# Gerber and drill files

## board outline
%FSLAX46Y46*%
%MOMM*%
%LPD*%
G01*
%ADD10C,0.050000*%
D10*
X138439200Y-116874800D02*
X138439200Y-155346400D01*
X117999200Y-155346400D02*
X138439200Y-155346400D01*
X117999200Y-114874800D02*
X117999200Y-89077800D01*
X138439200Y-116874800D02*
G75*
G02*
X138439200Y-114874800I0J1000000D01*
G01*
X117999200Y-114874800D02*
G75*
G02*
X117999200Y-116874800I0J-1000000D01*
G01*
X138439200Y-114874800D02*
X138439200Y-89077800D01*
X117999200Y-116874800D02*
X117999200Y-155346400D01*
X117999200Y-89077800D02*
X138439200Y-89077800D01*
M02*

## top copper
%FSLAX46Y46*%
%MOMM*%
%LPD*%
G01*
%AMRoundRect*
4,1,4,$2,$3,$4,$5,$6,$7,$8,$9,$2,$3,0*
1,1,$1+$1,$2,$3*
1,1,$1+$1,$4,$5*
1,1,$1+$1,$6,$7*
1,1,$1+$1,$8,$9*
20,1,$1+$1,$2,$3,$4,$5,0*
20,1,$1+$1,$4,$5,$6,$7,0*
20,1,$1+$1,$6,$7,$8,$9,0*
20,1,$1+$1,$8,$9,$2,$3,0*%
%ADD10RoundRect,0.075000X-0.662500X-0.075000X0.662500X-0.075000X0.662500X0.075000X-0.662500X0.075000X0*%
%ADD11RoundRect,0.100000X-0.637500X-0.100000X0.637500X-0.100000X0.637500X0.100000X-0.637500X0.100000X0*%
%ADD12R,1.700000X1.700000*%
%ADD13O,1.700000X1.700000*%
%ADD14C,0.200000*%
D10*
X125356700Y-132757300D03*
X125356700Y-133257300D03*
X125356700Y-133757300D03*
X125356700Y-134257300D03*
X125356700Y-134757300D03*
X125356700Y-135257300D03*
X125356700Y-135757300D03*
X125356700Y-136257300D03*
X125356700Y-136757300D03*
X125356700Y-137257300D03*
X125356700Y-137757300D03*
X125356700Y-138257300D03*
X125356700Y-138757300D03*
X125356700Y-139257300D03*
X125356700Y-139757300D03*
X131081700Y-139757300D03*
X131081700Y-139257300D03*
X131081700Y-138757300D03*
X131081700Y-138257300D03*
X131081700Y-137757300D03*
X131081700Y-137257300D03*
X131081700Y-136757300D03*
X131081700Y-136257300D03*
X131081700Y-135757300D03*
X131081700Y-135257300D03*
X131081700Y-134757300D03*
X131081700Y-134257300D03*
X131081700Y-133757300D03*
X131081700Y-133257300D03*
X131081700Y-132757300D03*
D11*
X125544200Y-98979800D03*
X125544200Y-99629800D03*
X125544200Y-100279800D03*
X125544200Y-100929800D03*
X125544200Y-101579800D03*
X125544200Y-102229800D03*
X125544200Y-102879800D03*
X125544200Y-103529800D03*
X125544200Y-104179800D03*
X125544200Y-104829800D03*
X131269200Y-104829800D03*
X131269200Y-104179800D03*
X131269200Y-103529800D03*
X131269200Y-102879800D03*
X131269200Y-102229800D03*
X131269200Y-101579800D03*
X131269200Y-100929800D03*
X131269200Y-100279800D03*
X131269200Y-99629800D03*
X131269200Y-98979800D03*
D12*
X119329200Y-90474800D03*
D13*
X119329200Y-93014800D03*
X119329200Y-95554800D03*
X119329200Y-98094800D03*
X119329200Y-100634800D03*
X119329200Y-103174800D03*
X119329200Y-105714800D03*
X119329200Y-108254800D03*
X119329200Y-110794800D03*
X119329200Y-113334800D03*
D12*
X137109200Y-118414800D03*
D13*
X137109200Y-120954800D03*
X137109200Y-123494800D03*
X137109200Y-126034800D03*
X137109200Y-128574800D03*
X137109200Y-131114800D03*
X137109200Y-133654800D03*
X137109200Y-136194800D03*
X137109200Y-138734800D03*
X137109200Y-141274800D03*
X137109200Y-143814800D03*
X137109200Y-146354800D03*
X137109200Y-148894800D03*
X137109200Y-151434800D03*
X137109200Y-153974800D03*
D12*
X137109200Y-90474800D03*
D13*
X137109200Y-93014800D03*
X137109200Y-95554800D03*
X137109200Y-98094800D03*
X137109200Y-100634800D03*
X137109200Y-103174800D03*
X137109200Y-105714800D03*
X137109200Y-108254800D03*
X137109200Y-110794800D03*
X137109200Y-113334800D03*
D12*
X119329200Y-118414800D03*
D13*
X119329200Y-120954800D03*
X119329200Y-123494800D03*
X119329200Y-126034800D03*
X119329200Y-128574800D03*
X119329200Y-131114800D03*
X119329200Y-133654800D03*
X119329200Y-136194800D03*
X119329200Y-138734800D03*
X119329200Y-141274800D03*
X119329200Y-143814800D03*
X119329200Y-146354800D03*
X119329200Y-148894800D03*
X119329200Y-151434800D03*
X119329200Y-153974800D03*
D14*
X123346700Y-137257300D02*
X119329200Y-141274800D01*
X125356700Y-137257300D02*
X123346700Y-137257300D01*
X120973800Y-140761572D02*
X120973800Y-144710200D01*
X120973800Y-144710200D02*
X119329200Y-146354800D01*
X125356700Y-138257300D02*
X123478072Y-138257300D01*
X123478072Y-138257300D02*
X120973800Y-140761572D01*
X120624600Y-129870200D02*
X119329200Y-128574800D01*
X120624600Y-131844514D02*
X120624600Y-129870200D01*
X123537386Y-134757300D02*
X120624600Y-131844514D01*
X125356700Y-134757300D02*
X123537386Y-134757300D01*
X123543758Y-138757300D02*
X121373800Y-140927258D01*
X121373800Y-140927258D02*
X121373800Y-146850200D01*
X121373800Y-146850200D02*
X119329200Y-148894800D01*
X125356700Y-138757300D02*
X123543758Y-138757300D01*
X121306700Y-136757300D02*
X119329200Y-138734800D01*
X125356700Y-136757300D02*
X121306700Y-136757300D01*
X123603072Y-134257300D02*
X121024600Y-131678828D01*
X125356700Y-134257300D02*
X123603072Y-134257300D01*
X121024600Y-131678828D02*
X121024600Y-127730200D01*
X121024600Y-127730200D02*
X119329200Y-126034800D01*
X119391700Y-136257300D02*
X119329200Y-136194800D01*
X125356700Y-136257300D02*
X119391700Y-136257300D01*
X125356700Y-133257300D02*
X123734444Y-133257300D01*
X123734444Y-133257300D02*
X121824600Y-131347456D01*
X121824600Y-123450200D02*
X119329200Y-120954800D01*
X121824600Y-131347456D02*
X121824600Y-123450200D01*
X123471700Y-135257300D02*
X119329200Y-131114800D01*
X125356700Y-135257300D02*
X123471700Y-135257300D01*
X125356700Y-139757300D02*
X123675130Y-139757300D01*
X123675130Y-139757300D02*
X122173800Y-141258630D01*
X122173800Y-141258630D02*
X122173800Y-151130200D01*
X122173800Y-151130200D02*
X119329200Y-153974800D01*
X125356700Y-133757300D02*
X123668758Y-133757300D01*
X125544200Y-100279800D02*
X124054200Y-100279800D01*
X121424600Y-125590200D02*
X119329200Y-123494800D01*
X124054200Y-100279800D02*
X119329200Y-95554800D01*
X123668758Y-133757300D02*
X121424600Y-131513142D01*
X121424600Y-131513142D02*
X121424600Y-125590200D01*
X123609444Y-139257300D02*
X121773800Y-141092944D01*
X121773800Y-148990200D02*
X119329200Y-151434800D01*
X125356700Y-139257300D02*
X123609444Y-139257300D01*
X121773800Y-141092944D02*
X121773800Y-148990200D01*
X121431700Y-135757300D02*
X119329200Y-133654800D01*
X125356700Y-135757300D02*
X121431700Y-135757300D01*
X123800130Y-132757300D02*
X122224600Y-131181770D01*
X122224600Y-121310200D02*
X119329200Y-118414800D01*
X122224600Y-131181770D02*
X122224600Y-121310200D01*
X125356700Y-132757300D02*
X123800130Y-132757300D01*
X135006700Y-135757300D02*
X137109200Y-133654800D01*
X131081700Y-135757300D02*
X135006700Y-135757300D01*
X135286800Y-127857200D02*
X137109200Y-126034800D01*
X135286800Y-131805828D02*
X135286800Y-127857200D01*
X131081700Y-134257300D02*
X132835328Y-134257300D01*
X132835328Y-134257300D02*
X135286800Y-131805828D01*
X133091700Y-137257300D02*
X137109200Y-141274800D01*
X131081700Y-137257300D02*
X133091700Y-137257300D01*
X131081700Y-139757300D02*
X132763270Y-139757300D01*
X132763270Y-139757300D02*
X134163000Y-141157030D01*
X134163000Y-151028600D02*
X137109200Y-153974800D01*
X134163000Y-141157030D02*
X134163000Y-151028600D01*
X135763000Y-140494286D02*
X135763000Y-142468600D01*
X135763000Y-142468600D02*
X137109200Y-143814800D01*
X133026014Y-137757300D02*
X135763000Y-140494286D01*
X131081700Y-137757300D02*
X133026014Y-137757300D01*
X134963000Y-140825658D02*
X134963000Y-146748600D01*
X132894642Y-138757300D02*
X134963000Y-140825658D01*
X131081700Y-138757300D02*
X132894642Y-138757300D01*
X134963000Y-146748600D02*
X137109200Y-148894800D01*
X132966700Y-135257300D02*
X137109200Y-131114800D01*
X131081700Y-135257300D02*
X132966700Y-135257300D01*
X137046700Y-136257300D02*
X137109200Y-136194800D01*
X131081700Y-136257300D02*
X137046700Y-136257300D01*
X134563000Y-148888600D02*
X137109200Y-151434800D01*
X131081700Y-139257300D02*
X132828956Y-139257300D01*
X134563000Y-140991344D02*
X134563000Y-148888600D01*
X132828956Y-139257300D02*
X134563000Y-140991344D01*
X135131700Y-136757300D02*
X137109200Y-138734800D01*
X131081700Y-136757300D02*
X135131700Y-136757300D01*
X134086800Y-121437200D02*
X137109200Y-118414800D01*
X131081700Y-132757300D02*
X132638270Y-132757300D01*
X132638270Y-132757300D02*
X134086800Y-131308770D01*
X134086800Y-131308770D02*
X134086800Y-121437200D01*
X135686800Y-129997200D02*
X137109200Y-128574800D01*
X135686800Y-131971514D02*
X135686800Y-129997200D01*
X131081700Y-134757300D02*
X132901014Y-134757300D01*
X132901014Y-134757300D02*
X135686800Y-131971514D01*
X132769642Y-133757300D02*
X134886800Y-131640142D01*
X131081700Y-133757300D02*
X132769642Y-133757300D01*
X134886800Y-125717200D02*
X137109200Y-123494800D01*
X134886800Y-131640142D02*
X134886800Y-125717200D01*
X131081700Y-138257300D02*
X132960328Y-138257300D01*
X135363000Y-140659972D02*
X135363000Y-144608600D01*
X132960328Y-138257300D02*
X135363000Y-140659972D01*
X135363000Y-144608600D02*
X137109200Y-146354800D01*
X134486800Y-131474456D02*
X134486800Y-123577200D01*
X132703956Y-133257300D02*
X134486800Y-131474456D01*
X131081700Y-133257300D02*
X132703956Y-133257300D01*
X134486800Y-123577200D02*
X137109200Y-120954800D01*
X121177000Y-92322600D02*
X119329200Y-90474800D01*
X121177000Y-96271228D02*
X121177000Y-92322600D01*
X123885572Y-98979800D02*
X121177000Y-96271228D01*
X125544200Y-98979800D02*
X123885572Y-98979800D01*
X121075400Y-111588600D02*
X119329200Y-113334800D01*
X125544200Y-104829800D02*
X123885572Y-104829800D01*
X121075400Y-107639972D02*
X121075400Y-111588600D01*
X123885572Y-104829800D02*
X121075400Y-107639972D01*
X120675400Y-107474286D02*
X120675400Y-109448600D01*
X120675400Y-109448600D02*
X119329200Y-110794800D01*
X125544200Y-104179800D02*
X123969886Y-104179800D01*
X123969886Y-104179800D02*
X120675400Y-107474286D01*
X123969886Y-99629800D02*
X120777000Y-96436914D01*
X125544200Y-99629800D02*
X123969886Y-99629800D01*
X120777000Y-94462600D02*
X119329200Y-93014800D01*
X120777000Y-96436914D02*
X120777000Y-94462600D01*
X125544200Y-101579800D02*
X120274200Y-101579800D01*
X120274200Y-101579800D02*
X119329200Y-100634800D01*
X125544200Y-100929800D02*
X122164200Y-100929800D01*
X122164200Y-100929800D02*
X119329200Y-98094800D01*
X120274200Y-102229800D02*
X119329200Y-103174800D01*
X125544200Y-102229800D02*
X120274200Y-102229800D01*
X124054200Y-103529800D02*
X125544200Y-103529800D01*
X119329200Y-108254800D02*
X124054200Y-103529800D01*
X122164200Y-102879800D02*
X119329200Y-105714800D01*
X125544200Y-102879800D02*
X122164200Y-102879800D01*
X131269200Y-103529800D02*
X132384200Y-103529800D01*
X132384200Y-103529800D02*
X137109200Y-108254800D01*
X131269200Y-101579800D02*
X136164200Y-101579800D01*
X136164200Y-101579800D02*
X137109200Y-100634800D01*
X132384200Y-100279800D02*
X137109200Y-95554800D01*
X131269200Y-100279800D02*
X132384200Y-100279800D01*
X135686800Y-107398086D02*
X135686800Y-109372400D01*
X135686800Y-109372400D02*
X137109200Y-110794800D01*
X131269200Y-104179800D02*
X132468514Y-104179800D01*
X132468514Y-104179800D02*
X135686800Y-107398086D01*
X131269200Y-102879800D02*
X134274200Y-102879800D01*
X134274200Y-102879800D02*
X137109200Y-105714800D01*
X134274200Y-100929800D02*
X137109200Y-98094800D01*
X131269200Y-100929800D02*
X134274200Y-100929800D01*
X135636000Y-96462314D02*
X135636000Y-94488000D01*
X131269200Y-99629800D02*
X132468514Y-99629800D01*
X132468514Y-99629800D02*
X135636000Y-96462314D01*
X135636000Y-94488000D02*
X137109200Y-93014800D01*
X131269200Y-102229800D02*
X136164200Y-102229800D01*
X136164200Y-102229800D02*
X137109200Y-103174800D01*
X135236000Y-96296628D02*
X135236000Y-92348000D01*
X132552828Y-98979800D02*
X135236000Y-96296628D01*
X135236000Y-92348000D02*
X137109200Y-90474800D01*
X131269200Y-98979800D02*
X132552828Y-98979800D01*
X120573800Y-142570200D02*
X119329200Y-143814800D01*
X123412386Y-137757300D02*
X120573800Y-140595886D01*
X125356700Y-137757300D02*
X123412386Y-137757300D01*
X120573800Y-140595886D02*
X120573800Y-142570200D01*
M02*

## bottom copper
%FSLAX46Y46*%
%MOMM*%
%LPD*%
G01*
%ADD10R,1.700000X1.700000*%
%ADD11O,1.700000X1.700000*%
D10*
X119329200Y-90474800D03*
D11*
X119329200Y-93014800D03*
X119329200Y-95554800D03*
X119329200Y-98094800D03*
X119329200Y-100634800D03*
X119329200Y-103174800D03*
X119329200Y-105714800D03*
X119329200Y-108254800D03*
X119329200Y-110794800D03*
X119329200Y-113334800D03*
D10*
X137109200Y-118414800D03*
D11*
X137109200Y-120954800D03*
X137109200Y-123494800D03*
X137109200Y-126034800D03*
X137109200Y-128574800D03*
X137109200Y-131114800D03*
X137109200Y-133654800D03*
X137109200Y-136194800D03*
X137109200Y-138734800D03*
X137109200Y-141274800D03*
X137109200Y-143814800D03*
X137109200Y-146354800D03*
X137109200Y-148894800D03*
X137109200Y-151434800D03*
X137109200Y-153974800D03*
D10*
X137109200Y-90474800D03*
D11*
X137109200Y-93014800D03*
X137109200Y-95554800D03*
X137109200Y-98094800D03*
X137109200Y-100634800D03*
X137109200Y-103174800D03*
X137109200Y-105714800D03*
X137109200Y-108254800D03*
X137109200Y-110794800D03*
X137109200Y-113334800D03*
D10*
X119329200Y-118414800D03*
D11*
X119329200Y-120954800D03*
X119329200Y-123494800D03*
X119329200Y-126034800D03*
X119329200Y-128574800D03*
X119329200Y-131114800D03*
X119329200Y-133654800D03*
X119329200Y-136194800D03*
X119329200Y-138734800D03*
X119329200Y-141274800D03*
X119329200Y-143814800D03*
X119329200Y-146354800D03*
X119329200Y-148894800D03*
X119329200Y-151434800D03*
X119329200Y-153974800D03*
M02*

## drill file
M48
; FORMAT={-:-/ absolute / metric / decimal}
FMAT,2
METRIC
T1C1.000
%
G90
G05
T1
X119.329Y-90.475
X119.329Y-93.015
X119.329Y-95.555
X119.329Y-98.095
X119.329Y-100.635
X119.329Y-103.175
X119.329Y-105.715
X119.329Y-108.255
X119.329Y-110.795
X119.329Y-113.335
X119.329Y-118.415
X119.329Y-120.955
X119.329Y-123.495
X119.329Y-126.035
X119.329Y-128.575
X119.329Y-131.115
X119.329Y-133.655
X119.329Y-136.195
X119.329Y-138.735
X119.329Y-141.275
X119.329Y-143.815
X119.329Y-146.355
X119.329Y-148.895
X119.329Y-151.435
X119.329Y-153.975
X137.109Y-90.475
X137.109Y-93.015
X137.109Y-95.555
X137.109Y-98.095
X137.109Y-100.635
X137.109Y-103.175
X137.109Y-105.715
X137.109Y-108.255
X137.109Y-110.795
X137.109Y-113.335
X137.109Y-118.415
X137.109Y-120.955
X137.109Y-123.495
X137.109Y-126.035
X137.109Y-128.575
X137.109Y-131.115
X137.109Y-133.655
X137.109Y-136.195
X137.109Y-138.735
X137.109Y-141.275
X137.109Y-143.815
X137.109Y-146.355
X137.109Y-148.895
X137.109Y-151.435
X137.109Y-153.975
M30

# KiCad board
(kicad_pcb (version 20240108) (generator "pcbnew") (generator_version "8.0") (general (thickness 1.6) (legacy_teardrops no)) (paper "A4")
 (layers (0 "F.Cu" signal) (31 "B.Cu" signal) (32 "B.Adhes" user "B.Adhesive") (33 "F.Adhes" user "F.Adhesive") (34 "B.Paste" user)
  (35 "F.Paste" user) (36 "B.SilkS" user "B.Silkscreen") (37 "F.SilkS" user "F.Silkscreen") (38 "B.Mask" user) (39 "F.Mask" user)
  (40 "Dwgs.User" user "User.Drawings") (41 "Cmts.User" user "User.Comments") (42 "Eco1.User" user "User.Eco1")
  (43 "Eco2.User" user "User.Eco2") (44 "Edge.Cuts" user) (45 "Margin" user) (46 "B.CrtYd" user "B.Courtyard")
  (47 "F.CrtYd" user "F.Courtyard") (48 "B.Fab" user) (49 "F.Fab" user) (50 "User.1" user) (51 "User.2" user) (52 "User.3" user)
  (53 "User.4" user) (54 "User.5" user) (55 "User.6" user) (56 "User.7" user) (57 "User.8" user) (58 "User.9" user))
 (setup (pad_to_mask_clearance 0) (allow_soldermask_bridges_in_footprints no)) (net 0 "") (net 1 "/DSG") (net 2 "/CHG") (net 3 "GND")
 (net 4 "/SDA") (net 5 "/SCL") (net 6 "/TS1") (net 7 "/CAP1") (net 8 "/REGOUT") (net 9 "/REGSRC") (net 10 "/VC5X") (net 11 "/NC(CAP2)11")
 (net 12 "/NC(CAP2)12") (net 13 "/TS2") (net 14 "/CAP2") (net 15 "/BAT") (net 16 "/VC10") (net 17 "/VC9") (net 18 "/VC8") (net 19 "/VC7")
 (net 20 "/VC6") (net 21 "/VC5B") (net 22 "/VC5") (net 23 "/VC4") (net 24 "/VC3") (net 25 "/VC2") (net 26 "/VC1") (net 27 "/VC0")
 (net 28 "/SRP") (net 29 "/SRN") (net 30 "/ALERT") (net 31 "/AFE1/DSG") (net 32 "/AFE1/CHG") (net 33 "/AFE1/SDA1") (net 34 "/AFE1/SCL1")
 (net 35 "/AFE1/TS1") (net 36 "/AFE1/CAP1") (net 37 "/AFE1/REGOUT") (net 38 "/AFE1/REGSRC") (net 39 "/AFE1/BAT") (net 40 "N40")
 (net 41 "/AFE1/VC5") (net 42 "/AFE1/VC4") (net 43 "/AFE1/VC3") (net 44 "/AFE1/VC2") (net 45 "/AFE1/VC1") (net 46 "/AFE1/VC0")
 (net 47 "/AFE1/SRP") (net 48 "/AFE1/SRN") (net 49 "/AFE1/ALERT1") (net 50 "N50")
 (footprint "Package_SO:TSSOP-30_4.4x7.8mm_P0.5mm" (layer "F.Cu") (at 128.2192 136.2573)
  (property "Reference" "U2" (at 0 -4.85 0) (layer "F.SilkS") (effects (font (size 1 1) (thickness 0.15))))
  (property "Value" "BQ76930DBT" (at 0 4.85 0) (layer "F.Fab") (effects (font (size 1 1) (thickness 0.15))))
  (pad "1" smd roundrect (at -2.8625 -3.5) (size 1.475 0.3) (layers "F.Cu" "F.Paste" "F.Mask") (roundrect_rratio 0.25) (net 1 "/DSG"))
  (pad "2" smd roundrect (at -2.8625 -3) (size 1.475 0.3) (layers "F.Cu" "F.Paste" "F.Mask") (roundrect_rratio 0.25) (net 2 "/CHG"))
  (pad "3" smd roundrect (at -2.8625 -2.5) (size 1.475 0.3) (layers "F.Cu" "F.Paste" "F.Mask") (roundrect_rratio 0.25) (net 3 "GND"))
  (pad "4" smd roundrect (at -2.8625 -2) (size 1.475 0.3) (layers "F.Cu" "F.Paste" "F.Mask") (roundrect_rratio 0.25) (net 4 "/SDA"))
  (pad "5" smd roundrect (at -2.8625 -1.5) (size 1.475 0.3) (layers "F.Cu" "F.Paste" "F.Mask") (roundrect_rratio 0.25) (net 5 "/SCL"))
  (pad "6" smd roundrect (at -2.8625 -1) (size 1.475 0.3) (layers "F.Cu" "F.Paste" "F.Mask") (roundrect_rratio 0.25) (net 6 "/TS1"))
  (pad "7" smd roundrect (at -2.8625 -0.5) (size 1.475 0.3) (layers "F.Cu" "F.Paste" "F.Mask") (roundrect_rratio 0.25) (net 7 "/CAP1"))
  (pad "8" smd roundrect (at -2.8625 0) (size 1.475 0.3) (layers "F.Cu" "F.Paste" "F.Mask") (roundrect_rratio 0.25) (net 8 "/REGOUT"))
  (pad "9" smd roundrect (at -2.8625 0.5) (size 1.475 0.3) (layers "F.Cu" "F.Paste" "F.Mask") (roundrect_rratio 0.25) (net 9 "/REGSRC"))
  (pad "10" smd roundrect (at -2.8625 1) (size 1.475 0.3) (layers "F.Cu" "F.Paste" "F.Mask") (roundrect_rratio 0.25) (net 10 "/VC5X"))
  (pad "11" smd roundrect (at -2.8625 1.5) (size 1.475 0.3) (layers "F.Cu" "F.Paste" "F.Mask") (roundrect_rratio 0.25)
   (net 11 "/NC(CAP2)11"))
  (pad "12" smd roundrect (at -2.8625 2) (size 1.475 0.3) (layers "F.Cu" "F.Paste" "F.Mask") (roundrect_rratio 0.25) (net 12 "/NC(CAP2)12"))
  (pad "13" smd roundrect (at -2.8625 2.5) (size 1.475 0.3) (layers "F.Cu" "F.Paste" "F.Mask") (roundrect_rratio 0.25) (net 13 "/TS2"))
  (pad "14" smd roundrect (at -2.8625 3) (size 1.475 0.3) (layers "F.Cu" "F.Paste" "F.Mask") (roundrect_rratio 0.25) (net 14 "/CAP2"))
  (pad "15" smd roundrect (at -2.8625 3.5) (size 1.475 0.3) (layers "F.Cu" "F.Paste" "F.Mask") (roundrect_rratio 0.25) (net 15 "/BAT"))
  (pad "16" smd roundrect (at 2.8625 3.5) (size 1.475 0.3) (layers "F.Cu" "F.Paste" "F.Mask") (roundrect_rratio 0.25) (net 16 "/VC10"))
  (pad "17" smd roundrect (at 2.8625 3) (size 1.475 0.3) (layers "F.Cu" "F.Paste" "F.Mask") (roundrect_rratio 0.25) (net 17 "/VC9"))
  (pad "18" smd roundrect (at 2.8625 2.5) (size 1.475 0.3) (layers "F.Cu" "F.Paste" "F.Mask") (roundrect_rratio 0.25) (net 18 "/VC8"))
  (pad "19" smd roundrect (at 2.8625 2) (size 1.475 0.3) (layers "F.Cu" "F.Paste" "F.Mask") (roundrect_rratio 0.25) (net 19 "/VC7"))
  (pad "20" smd roundrect (at 2.8625 1.5) (size 1.475 0.3) (layers "F.Cu" "F.Paste" "F.Mask") (roundrect_rratio 0.25) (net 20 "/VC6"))
  (pad "21" smd roundrect (at 2.8625 1) (size 1.475 0.3) (layers "F.Cu" "F.Paste" "F.Mask") (roundrect_rratio 0.25) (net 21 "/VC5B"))
  (pad "22" smd roundrect (at 2.8625 0.5) (size 1.475 0.3) (layers "F.Cu" "F.Paste" "F.Mask") (roundrect_rratio 0.25) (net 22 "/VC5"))
  (pad "23" smd roundrect (at 2.8625 0) (size 1.475 0.3) (layers "F.Cu" "F.Paste" "F.Mask") (roundrect_rratio 0.25) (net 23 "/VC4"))
  (pad "24" smd roundrect (at 2.8625 -0.5) (size 1.475 0.3) (layers "F.Cu" "F.Paste" "F.Mask") (roundrect_rratio 0.25) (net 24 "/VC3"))
  (pad "25" smd roundrect (at 2.8625 -1) (size 1.475 0.3) (layers "F.Cu" "F.Paste" "F.Mask") (roundrect_rratio 0.25) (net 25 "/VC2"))
  (pad "26" smd roundrect (at 2.8625 -1.5) (size 1.475 0.3) (layers "F.Cu" "F.Paste" "F.Mask") (roundrect_rratio 0.25) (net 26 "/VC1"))
  (pad "27" smd roundrect (at 2.8625 -2) (size 1.475 0.3) (layers "F.Cu" "F.Paste" "F.Mask") (roundrect_rratio 0.25) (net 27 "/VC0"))
  (pad "28" smd roundrect (at 2.8625 -2.5) (size 1.475 0.3) (layers "F.Cu" "F.Paste" "F.Mask") (roundrect_rratio 0.25) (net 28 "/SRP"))
  (pad "29" smd roundrect (at 2.8625 -3) (size 1.475 0.3) (layers "F.Cu" "F.Paste" "F.Mask") (roundrect_rratio 0.25) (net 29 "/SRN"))
  (pad "30" smd roundrect (at 2.8625 -3.5) (size 1.475 0.3) (layers "F.Cu" "F.Paste" "F.Mask") (roundrect_rratio 0.25) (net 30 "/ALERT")))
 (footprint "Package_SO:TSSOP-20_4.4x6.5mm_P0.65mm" (layer "F.Cu") (at 128.4067 101.9048)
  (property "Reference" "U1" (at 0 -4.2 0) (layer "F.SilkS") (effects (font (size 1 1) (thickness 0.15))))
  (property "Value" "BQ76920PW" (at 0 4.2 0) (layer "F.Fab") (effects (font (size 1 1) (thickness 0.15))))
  (pad "1" smd roundrect (at -2.8625 -2.925) (size 1.475 0.4) (layers "F.Cu" "F.Paste" "F.Mask") (roundrect_rratio 0.25)
   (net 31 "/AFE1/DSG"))
  (pad "2" smd roundrect (at -2.8625 -2.275) (size 1.475 0.4) (layers "F.Cu" "F.Paste" "F.Mask") (roundrect_rratio 0.25)
   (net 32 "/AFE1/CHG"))
  (pad "3" smd roundrect (at -2.8625 -1.625) (size 1.475 0.4) (layers "F.Cu" "F.Paste" "F.Mask") (roundrect_rratio 0.25) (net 3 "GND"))
  (pad "4" smd roundrect (at -2.8625 -0.975) (size 1.475 0.4) (layers "F.Cu" "F.Paste" "F.Mask") (roundrect_rratio 0.25)
   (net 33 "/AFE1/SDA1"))
  (pad "5" smd roundrect (at -2.8625 -0.325) (size 1.475 0.4) (layers "F.Cu" "F.Paste" "F.Mask") (roundrect_rratio 0.25)
   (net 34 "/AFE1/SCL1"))
  (pad "6" smd roundrect (at -2.8625 0.325) (size 1.475 0.4) (layers "F.Cu" "F.Paste" "F.Mask") (roundrect_rratio 0.25) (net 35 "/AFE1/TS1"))
  (pad "7" smd roundrect (at -2.8625 0.975) (size 1.475 0.4) (layers "F.Cu" "F.Paste" "F.Mask") (roundrect_rratio 0.25)
   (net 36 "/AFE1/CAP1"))
  (pad "8" smd roundrect (at -2.8625 1.625) (size 1.475 0.4) (layers "F.Cu" "F.Paste" "F.Mask") (roundrect_rratio 0.25)
   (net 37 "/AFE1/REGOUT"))
  (pad "9" smd roundrect (at -2.8625 2.275) (size 1.475 0.4) (layers "F.Cu" "F.Paste" "F.Mask") (roundrect_rratio 0.25)
   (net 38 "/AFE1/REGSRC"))
  (pad "10" smd roundrect (at -2.8625 2.925) (size 1.475 0.4) (layers "F.Cu" "F.Paste" "F.Mask") (roundrect_rratio 0.25)
   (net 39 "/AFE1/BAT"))
  (pad "11" smd roundrect (at 2.8625 2.925) (size 1.475 0.4) (layers "F.Cu" "F.Paste" "F.Mask") (roundrect_rratio 0.25) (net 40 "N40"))
  (pad "12" smd roundrect (at 2.8625 2.275) (size 1.475 0.4) (layers "F.Cu" "F.Paste" "F.Mask") (roundrect_rratio 0.25) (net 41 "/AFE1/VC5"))
  (pad "13" smd roundrect (at 2.8625 1.625) (size 1.475 0.4) (layers "F.Cu" "F.Paste" "F.Mask") (roundrect_rratio 0.25) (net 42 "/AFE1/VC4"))
  (pad "14" smd roundrect (at 2.8625 0.975) (size 1.475 0.4) (layers "F.Cu" "F.Paste" "F.Mask") (roundrect_rratio 0.25) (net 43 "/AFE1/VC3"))
  (pad "15" smd roundrect (at 2.8625 0.325) (size 1.475 0.4) (layers "F.Cu" "F.Paste" "F.Mask") (roundrect_rratio 0.25) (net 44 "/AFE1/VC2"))
  (pad "16" smd roundrect (at 2.8625 -0.325) (size 1.475 0.4) (layers "F.Cu" "F.Paste" "F.Mask") (roundrect_rratio 0.25)
   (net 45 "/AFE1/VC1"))
  (pad "17" smd roundrect (at 2.8625 -0.975) (size 1.475 0.4) (layers "F.Cu" "F.Paste" "F.Mask") (roundrect_rratio 0.25)
   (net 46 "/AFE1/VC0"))
  (pad "18" smd roundrect (at 2.8625 -1.625) (size 1.475 0.4) (layers "F.Cu" "F.Paste" "F.Mask") (roundrect_rratio 0.25)
   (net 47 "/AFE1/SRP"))
  (pad "19" smd roundrect (at 2.8625 -2.275) (size 1.475 0.4) (layers "F.Cu" "F.Paste" "F.Mask") (roundrect_rratio 0.25)
   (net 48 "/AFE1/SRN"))
  (pad "20" smd roundrect (at 2.8625 -2.925) (size 1.475 0.4) (layers "F.Cu" "F.Paste" "F.Mask") (roundrect_rratio 0.25)
   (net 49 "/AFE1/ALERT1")))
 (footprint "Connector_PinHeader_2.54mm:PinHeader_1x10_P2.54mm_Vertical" (layer "B.Cu") (at 119.3292 90.4748 180)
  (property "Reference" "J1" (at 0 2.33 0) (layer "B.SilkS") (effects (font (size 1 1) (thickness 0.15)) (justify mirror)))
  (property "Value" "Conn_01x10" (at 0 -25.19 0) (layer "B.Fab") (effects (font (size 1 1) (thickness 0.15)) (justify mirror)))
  (pad "1" thru_hole rect (at 0 0 180) (size 1.7 1.7) (drill 1) (layers "*.Cu" "*.Mask") (remove_unused_layers no) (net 31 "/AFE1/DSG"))
  (pad "2" thru_hole oval (at 0 -2.54 180) (size 1.7 1.7) (drill 1) (layers "*.Cu" "*.Mask") (remove_unused_layers no) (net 32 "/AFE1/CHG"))
  (pad "3" thru_hole oval (at 0 -5.08 180) (size 1.7 1.7) (drill 1) (layers "*.Cu" "*.Mask") (remove_unused_layers no) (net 3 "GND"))
  (pad "4" thru_hole oval (at 0 -7.62 180) (size 1.7 1.7) (drill 1) (layers "*.Cu" "*.Mask") (remove_unused_layers no) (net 33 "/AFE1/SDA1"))
  (pad "5" thru_hole oval (at 0 -10.16 180) (size 1.7 1.7) (drill 1) (layers "*.Cu" "*.Mask") (remove_unused_layers no)
   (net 34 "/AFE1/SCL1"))
  (pad "6" thru_hole oval (at 0 -12.7 180) (size 1.7 1.7) (drill 1) (layers "*.Cu" "*.Mask") (remove_unused_layers no) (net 35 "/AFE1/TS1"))
  (pad "7" thru_hole oval (at 0 -15.24 180) (size 1.7 1.7) (drill 1) (layers "*.Cu" "*.Mask") (remove_unused_layers no)
   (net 36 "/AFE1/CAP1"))
  (pad "8" thru_hole oval (at 0 -17.78 180) (size 1.7 1.7) (drill 1) (layers "*.Cu" "*.Mask") (remove_unused_layers no)
   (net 37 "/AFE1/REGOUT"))
  (pad "9" thru_hole oval (at 0 -20.32 180) (size 1.7 1.7) (drill 1) (layers "*.Cu" "*.Mask") (remove_unused_layers no)
   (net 38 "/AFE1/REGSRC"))
  (pad "10" thru_hole oval (at 0 -22.86 180) (size 1.7 1.7) (drill 1) (layers "*.Cu" "*.Mask") (remove_unused_layers no)
   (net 39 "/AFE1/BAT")))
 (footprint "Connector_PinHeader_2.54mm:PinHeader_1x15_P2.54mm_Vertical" (layer "B.Cu") (at 137.1092 118.4148 180)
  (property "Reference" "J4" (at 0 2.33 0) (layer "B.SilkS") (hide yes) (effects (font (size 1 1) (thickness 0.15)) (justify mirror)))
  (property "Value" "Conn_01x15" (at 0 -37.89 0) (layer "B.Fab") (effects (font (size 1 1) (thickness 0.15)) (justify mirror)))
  (pad "1" thru_hole rect (at 0 0 180) (size 1.7 1.7) (drill 1) (layers "*.Cu" "*.Mask") (remove_unused_layers no) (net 30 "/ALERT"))
  (pad "2" thru_hole oval (at 0 -2.54 180) (size 1.7 1.7) (drill 1) (layers "*.Cu" "*.Mask") (remove_unused_layers no) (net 29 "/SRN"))
  (pad "3" thru_hole oval (at 0 -5.08 180) (size 1.7 1.7) (drill 1) (layers "*.Cu" "*.Mask") (remove_unused_layers no) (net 28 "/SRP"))
  (pad "4" thru_hole oval (at 0 -7.62 180) (size 1.7 1.7) (drill 1) (layers "*.Cu" "*.Mask") (remove_unused_layers no) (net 27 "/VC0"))
  (pad "5" thru_hole oval (at 0 -10.16 180) (size 1.7 1.7) (drill 1) (layers "*.Cu" "*.Mask") (remove_unused_layers no) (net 26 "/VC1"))
  (pad "6" thru_hole oval (at 0 -12.7 180) (size 1.7 1.7) (drill 1) (layers "*.Cu" "*.Mask") (remove_unused_layers no) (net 25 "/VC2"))
  (pad "7" thru_hole oval (at 0 -15.24 180) (size 1.7 1.7) (drill 1) (layers "*.Cu" "*.Mask") (remove_unused_layers no) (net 24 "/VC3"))
  (pad "8" thru_hole oval (at 0 -17.78 180) (size 1.7 1.7) (drill 1) (layers "*.Cu" "*.Mask") (remove_unused_layers no) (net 23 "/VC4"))
  (pad "9" thru_hole oval (at 0 -20.32 180) (size 1.7 1.7) (drill 1) (layers "*.Cu" "*.Mask") (remove_unused_layers no) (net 22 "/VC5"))
  (pad "10" thru_hole oval (at 0 -22.86 180) (size 1.7 1.7) (drill 1) (layers "*.Cu" "*.Mask") (remove_unused_layers no) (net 21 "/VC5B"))
  (pad "11" thru_hole oval (at 0 -25.4 180) (size 1.7 1.7) (drill 1) (layers "*.Cu" "*.Mask") (remove_unused_layers no) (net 20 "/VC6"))
  (pad "12" thru_hole oval (at 0 -27.94 180) (size 1.7 1.7) (drill 1) (layers "*.Cu" "*.Mask") (remove_unused_layers no) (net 19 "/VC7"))
  (pad "13" thru_hole oval (at 0 -30.48 180) (size 1.7 1.7) (drill 1) (layers "*.Cu" "*.Mask") (remove_unused_layers no) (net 18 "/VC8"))
  (pad "14" thru_hole oval (at 0 -33.02 180) (size 1.7 1.7) (drill 1) (layers "*.Cu" "*.Mask") (remove_unused_layers no) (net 17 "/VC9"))
  (pad "15" thru_hole oval (at 0 -35.56 180) (size 1.7 1.7) (drill 1) (layers "*.Cu" "*.Mask") (remove_unused_layers no) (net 16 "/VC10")))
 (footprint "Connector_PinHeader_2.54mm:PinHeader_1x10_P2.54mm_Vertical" (layer "B.Cu") (at 137.1092 90.4748 180)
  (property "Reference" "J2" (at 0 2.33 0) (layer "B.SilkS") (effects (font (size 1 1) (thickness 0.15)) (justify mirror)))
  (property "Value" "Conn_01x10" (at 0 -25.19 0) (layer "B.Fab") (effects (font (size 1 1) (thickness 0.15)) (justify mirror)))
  (pad "1" thru_hole rect (at 0 0 180) (size 1.7 1.7) (drill 1) (layers "*.Cu" "*.Mask") (remove_unused_layers no) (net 49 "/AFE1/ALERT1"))
  (pad "2" thru_hole oval (at 0 -2.54 180) (size 1.7 1.7) (drill 1) (layers "*.Cu" "*.Mask") (remove_unused_layers no) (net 48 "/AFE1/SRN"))
  (pad "3" thru_hole oval (at 0 -5.08 180) (size 1.7 1.7) (drill 1) (layers "*.Cu" "*.Mask") (remove_unused_layers no) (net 47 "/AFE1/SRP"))
  (pad "4" thru_hole oval (at 0 -7.62 180) (size 1.7 1.7) (drill 1) (layers "*.Cu" "*.Mask") (remove_unused_layers no) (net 46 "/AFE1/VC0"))
  (pad "5" thru_hole oval (at 0 -10.16 180) (size 1.7 1.7) (drill 1) (layers "*.Cu" "*.Mask") (remove_unused_layers no) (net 45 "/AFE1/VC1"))
  (pad "6" thru_hole oval (at 0 -12.7 180) (size 1.7 1.7) (drill 1) (layers "*.Cu" "*.Mask") (remove_unused_layers no) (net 44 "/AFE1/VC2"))
  (pad "7" thru_hole oval (at 0 -15.24 180) (size 1.7 1.7) (drill 1) (layers "*.Cu" "*.Mask") (remove_unused_layers no) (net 43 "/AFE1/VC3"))
  (pad "8" thru_hole oval (at 0 -17.78 180) (size 1.7 1.7) (drill 1) (layers "*.Cu" "*.Mask") (remove_unused_layers no) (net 42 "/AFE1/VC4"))
  (pad "9" thru_hole oval (at 0 -20.32 180) (size 1.7 1.7) (drill 1) (layers "*.Cu" "*.Mask") (remove_unused_layers no) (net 41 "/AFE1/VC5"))
  (pad "10" thru_hole oval (at 0 -22.86 180) (size 1.7 1.7) (drill 1) (layers "*.Cu" "*.Mask") (remove_unused_layers no) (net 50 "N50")))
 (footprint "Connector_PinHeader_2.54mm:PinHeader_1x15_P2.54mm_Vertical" (layer "B.Cu") (at 119.3292 118.4148 180)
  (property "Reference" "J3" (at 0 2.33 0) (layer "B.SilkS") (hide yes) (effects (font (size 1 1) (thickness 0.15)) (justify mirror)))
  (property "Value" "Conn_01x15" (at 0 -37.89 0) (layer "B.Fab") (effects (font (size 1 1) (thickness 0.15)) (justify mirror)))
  (pad "1" thru_hole rect (at 0 0 180) (size 1.7 1.7) (drill 1) (layers "*.Cu" "*.Mask") (remove_unused_layers no) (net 1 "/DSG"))
  (pad "2" thru_hole oval (at 0 -2.54 180) (size 1.7 1.7) (drill 1) (layers "*.Cu" "*.Mask") (remove_unused_layers no) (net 2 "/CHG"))
  (pad "3" thru_hole oval (at 0 -5.08 180) (size 1.7 1.7) (drill 1) (layers "*.Cu" "*.Mask") (remove_unused_layers no) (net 3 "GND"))
  (pad "4" thru_hole oval (at 0 -7.62 180) (size 1.7 1.7) (drill 1) (layers "*.Cu" "*.Mask") (remove_unused_layers no) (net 4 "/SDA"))
  (pad "5" thru_hole oval (at 0 -10.16 180) (size 1.7 1.7) (drill 1) (layers "*.Cu" "*.Mask") (remove_unused_layers no) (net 5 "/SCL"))
  (pad "6" thru_hole oval (at 0 -12.7 180) (size 1.7 1.7) (drill 1) (layers "*.Cu" "*.Mask") (remove_unused_layers no) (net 6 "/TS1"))
  (pad "7" thru_hole oval (at 0 -15.24 180) (size 1.7 1.7) (drill 1) (layers "*.Cu" "*.Mask") (remove_unused_layers no) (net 7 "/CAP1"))
  (pad "8" thru_hole oval (at 0 -17.78 180) (size 1.7 1.7) (drill 1) (layers "*.Cu" "*.Mask") (remove_unused_layers no) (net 8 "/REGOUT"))
  (pad "9" thru_hole oval (at 0 -20.32 180) (size 1.7 1.7) (drill 1) (layers "*.Cu" "*.Mask") (remove_unused_layers no) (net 9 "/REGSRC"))
  (pad "10" thru_hole oval (at 0 -22.86 180) (size 1.7 1.7) (drill 1) (layers "*.Cu" "*.Mask") (remove_unused_layers no) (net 10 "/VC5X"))
  (pad "11" thru_hole oval (at 0 -25.4 180) (size 1.7 1.7) (drill 1) (layers "*.Cu" "*.Mask") (remove_unused_layers no)
   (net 11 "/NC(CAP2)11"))
  (pad "12" thru_hole oval (at 0 -27.94 180) (size 1.7 1.7) (drill 1) (layers "*.Cu" "*.Mask") (remove_unused_layers no)
   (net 12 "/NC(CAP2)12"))
  (pad "13" thru_hole oval (at 0 -30.48 180) (size 1.7 1.7) (drill 1) (layers "*.Cu" "*.Mask") (remove_unused_layers no) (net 13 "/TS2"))
  (pad "14" thru_hole oval (at 0 -33.02 180) (size 1.7 1.7) (drill 1) (layers "*.Cu" "*.Mask") (remove_unused_layers no) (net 14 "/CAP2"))
  (pad "15" thru_hole oval (at 0 -35.56 180) (size 1.7 1.7) (drill 1) (layers "*.Cu" "*.Mask") (remove_unused_layers no) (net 15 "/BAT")))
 (gr_line (start 138.4392 116.8748) (end 138.4392 155.3464) (stroke (width 0.05) (type default)) (layer "Edge.Cuts"))
 (gr_line (start 117.9992 155.3464) (end 138.4392 155.3464) (stroke (width 0.05) (type default)) (layer "Edge.Cuts"))
 (gr_line (start 117.9992 114.8748) (end 117.9992 89.0778) (stroke (width 0.05) (type default)) (layer "Edge.Cuts"))
 (gr_arc (start 138.4392 116.8748) (mid 137.4392 115.8748) (end 138.4392 114.8748) (stroke (width 0.05) (type default)) (layer "Edge.Cuts"))
 (gr_arc (start 117.9992 114.8748) (mid 118.9992 115.8748) (end 117.9992 116.8748) (stroke (width 0.05) (type default)) (layer "Edge.Cuts"))
 (gr_line (start 138.4392 114.8748) (end 138.4392 89.0778) (stroke (width 0.05) (type default)) (layer "Edge.Cuts"))
 (gr_line (start 117.9992 116.8748) (end 117.9992 155.3464) (stroke (width 0.05) (type default)) (layer "Edge.Cuts"))
 (gr_line (start 117.9992 89.0778) (end 138.4392 89.0778) (stroke (width 0.05) (type default)) (layer "Edge.Cuts"))
 (segment (start 123.3467 137.2573) (end 119.3292 141.2748) (width 0.2) (layer "F.Cu") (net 10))
 (segment (start 125.3567 137.2573) (end 123.3467 137.2573) (width 0.2) (layer "F.Cu") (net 10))
 (segment (start 120.9738 140.761572) (end 120.9738 144.7102) (width 0.2) (layer "F.Cu") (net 12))
 (segment (start 120.9738 144.7102) (end 119.3292 146.3548) (width 0.2) (layer "F.Cu") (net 12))
 (segment (start 125.3567 138.2573) (end 123.478072 138.2573) (width 0.2) (layer "F.Cu") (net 12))
 (segment (start 123.478072 138.2573) (end 120.9738 140.761572) (width 0.2) (layer "F.Cu") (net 12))
 (segment (start 120.6246 129.8702) (end 119.3292 128.5748) (width 0.2) (layer "F.Cu") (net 5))
 (segment (start 120.6246 131.844514) (end 120.6246 129.8702) (width 0.2) (layer "F.Cu") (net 5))
 (segment (start 123.537386 134.7573) (end 120.6246 131.844514) (width 0.2) (layer "F.Cu") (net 5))
 (segment (start 125.3567 134.7573) (end 123.537386 134.7573) (width 0.2) (layer "F.Cu") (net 5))
 (segment (start 123.543758 138.7573) (end 121.3738 140.927258) (width 0.2) (layer "F.Cu") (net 13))
 (segment (start 121.3738 140.927258) (end 121.3738 146.8502) (width 0.2) (layer "F.Cu") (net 13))
 (segment (start 121.3738 146.8502) (end 119.3292 148.8948) (width 0.2) (layer "F.Cu") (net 13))
 (segment (start 125.3567 138.7573) (end 123.543758 138.7573) (width 0.2) (layer "F.Cu") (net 13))
 (segment (start 121.3067 136.7573) (end 119.3292 138.7348) (width 0.2) (layer "F.Cu") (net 9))
 (segment (start 125.3567 136.7573) (end 121.3067 136.7573) (width 0.2) (layer "F.Cu") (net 9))
 (segment (start 123.603072 134.2573) (end 121.0246 131.678828) (width 0.2) (layer "F.Cu") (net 4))
 (segment (start 125.3567 134.2573) (end 123.603072 134.2573) (width 0.2) (layer "F.Cu") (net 4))
 (segment (start 121.0246 131.678828) (end 121.0246 127.7302) (width 0.2) (layer "F.Cu") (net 4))
 (segment (start 121.0246 127.7302) (end 119.3292 126.0348) (width 0.2) (layer "F.Cu") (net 4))
 (segment (start 119.3917 136.2573) (end 119.3292 136.1948) (width 0.2) (layer "F.Cu") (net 8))
 (segment (start 125.3567 136.2573) (end 119.3917 136.2573) (width 0.2) (layer "F.Cu") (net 8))
 (segment (start 125.3567 133.2573) (end 123.734444 133.2573) (width 0.2) (layer "F.Cu") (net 2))
 (segment (start 123.734444 133.2573) (end 121.8246 131.347456) (width 0.2) (layer "F.Cu") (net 2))
 (segment (start 121.8246 123.4502) (end 119.3292 120.9548) (width 0.2) (layer "F.Cu") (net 2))
 (segment (start 121.8246 131.347456) (end 121.8246 123.4502) (width 0.2) (layer "F.Cu") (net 2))
 (segment (start 123.4717 135.2573) (end 119.3292 131.1148) (width 0.2) (layer "F.Cu") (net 6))
 (segment (start 125.3567 135.2573) (end 123.4717 135.2573) (width 0.2) (layer "F.Cu") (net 6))
 (segment (start 125.3567 139.7573) (end 123.67513 139.7573) (width 0.2) (layer "F.Cu") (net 15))
 (segment (start 123.67513 139.7573) (end 122.1738 141.25863) (width 0.2) (layer "F.Cu") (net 15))
 (segment (start 122.1738 141.25863) (end 122.1738 151.1302) (width 0.2) (layer "F.Cu") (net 15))
 (segment (start 122.1738 151.1302) (end 119.3292 153.9748) (width 0.2) (layer "F.Cu") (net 15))
 (segment (start 125.3567 133.7573) (end 123.668758 133.7573) (width 0.2) (layer "F.Cu") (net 3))
 (segment (start 125.5442 100.2798) (end 124.0542 100.2798) (width 0.2) (layer "F.Cu") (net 3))
 (segment (start 121.4246 125.5902) (end 119.3292 123.4948) (width 0.2) (layer "F.Cu") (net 3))
 (segment (start 124.0542 100.2798) (end 119.3292 95.5548) (width 0.2) (layer "F.Cu") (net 3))
 (segment (start 123.668758 133.7573) (end 121.4246 131.513142) (width 0.2) (layer "F.Cu") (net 3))
 (segment (start 121.4246 131.513142) (end 121.4246 125.5902) (width 0.2) (layer "F.Cu") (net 3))
 (segment (start 123.609444 139.2573) (end 121.7738 141.092944) (width 0.2) (layer "F.Cu") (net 14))
 (segment (start 121.7738 148.9902) (end 119.3292 151.4348) (width 0.2) (layer "F.Cu") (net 14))
 (segment (start 125.3567 139.2573) (end 123.609444 139.2573) (width 0.2) (layer "F.Cu") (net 14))
 (segment (start 121.7738 141.092944) (end 121.7738 148.9902) (width 0.2) (layer "F.Cu") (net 14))
 (segment (start 121.4317 135.7573) (end 119.3292 133.6548) (width 0.2) (layer "F.Cu") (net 7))
 (segment (start 125.3567 135.7573) (end 121.4317 135.7573) (width 0.2) (layer "F.Cu") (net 7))
 (segment (start 123.80013 132.7573) (end 122.2246 131.18177) (width 0.2) (layer "F.Cu") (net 1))
 (segment (start 122.2246 121.3102) (end 119.3292 118.4148) (width 0.2) (layer "F.Cu") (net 1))
 (segment (start 122.2246 131.18177) (end 122.2246 121.3102) (width 0.2) (layer "F.Cu") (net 1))
 (segment (start 125.3567 132.7573) (end 123.80013 132.7573) (width 0.2) (layer "F.Cu") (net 1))
 (segment (start 135.0067 135.7573) (end 137.1092 133.6548) (width 0.2) (layer "F.Cu") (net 24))
 (segment (start 131.0817 135.7573) (end 135.0067 135.7573) (width 0.2) (layer "F.Cu") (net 24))
 (segment (start 135.2868 127.8572) (end 137.1092 126.0348) (width 0.2) (layer "F.Cu") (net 27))
 (segment (start 135.2868 131.805828) (end 135.2868 127.8572) (width 0.2) (layer "F.Cu") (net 27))
 (segment (start 131.0817 134.2573) (end 132.835328 134.2573) (width 0.2) (layer "F.Cu") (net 27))
 (segment (start 132.835328 134.2573) (end 135.2868 131.805828) (width 0.2) (layer "F.Cu") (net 27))
 (segment (start 133.0917 137.2573) (end 137.1092 141.2748) (width 0.2) (layer "F.Cu") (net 21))
 (segment (start 131.0817 137.2573) (end 133.0917 137.2573) (width 0.2) (layer "F.Cu") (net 21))
 (segment (start 131.0817 139.7573) (end 132.76327 139.7573) (width 0.2) (layer "F.Cu") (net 16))
 (segment (start 132.76327 139.7573) (end 134.163 141.15703) (width 0.2) (layer "F.Cu") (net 16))
 (segment (start 134.163 151.0286) (end 137.1092 153.9748) (width 0.2) (layer "F.Cu") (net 16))
 (segment (start 134.163 141.15703) (end 134.163 151.0286) (width 0.2) (layer "F.Cu") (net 16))
 (segment (start 135.763 140.494286) (end 135.763 142.4686) (width 0.2) (layer "F.Cu") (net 20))
 (segment (start 135.763 142.4686) (end 137.1092 143.8148) (width 0.2) (layer "F.Cu") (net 20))
 (segment (start 133.026014 137.7573) (end 135.763 140.494286) (width 0.2) (layer "F.Cu") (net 20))
 (segment (start 131.0817 137.7573) (end 133.026014 137.7573) (width 0.2) (layer "F.Cu") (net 20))
 (segment (start 134.963 140.825658) (end 134.963 146.7486) (width 0.2) (layer "F.Cu") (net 18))
 (segment (start 132.894642 138.7573) (end 134.963 140.825658) (width 0.2) (layer "F.Cu") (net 18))
 (segment (start 131.0817 138.7573) (end 132.894642 138.7573) (width 0.2) (layer "F.Cu") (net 18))
 (segment (start 134.963 146.7486) (end 137.1092 148.8948) (width 0.2) (layer "F.Cu") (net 18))
 (segment (start 132.9667 135.2573) (end 137.1092 131.1148) (width 0.2) (layer "F.Cu") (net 25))
 (segment (start 131.0817 135.2573) (end 132.9667 135.2573) (width 0.2) (layer "F.Cu") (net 25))
 (segment (start 137.0467 136.2573) (end 137.1092 136.1948) (width 0.2) (layer "F.Cu") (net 23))
 (segment (start 131.0817 136.2573) (end 137.0467 136.2573) (width 0.2) (layer "F.Cu") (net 23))
 (segment (start 134.563 148.8886) (end 137.1092 151.4348) (width 0.2) (layer "F.Cu") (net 17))
 (segment (start 131.0817 139.2573) (end 132.828956 139.2573) (width 0.2) (layer "F.Cu") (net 17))
 (segment (start 134.563 140.991344) (end 134.563 148.8886) (width 0.2) (layer "F.Cu") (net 17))
 (segment (start 132.828956 139.2573) (end 134.563 140.991344) (width 0.2) (layer "F.Cu") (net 17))
 (segment (start 135.1317 136.7573) (end 137.1092 138.7348) (width 0.2) (layer "F.Cu") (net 22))
 (segment (start 131.0817 136.7573) (end 135.1317 136.7573) (width 0.2) (layer "F.Cu") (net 22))
 (segment (start 134.0868 121.4372) (end 137.1092 118.4148) (width 0.2) (layer "F.Cu") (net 30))
 (segment (start 131.0817 132.7573) (end 132.63827 132.7573) (width 0.2) (layer "F.Cu") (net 30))
 (segment (start 132.63827 132.7573) (end 134.0868 131.30877) (width 0.2) (layer "F.Cu") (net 30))
 (segment (start 134.0868 131.30877) (end 134.0868 121.4372) (width 0.2) (layer "F.Cu") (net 30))
 (segment (start 135.6868 129.9972) (end 137.1092 128.5748) (width 0.2) (layer "F.Cu") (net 26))
 (segment (start 135.6868 131.971514) (end 135.6868 129.9972) (width 0.2) (layer "F.Cu") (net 26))
 (segment (start 131.0817 134.7573) (end 132.901014 134.7573) (width 0.2) (layer "F.Cu") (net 26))
 (segment (start 132.901014 134.7573) (end 135.6868 131.971514) (width 0.2) (layer "F.Cu") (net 26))
 (segment (start 132.769642 133.7573) (end 134.8868 131.640142) (width 0.2) (layer "F.Cu") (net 28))
 (segment (start 131.0817 133.7573) (end 132.769642 133.7573) (width 0.2) (layer "F.Cu") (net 28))
 (segment (start 134.8868 125.7172) (end 137.1092 123.4948) (width 0.2) (layer "F.Cu") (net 28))
 (segment (start 134.8868 131.640142) (end 134.8868 125.7172) (width 0.2) (layer "F.Cu") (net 28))
 (segment (start 131.0817 138.2573) (end 132.960328 138.2573) (width 0.2) (layer "F.Cu") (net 19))
 (segment (start 135.363 140.659972) (end 135.363 144.6086) (width 0.2) (layer "F.Cu") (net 19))
 (segment (start 132.960328 138.2573) (end 135.363 140.659972) (width 0.2) (layer "F.Cu") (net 19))
 (segment (start 135.363 144.6086) (end 137.1092 146.3548) (width 0.2) (layer "F.Cu") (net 19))
 (segment (start 134.4868 131.474456) (end 134.4868 123.5772) (width 0.2) (layer "F.Cu") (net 29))
 (segment (start 132.703956 133.2573) (end 134.4868 131.474456) (width 0.2) (layer "F.Cu") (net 29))
 (segment (start 131.0817 133.2573) (end 132.703956 133.2573) (width 0.2) (layer "F.Cu") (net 29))
 (segment (start 134.4868 123.5772) (end 137.1092 120.9548) (width 0.2) (layer "F.Cu") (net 29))
 (segment (start 121.177 92.3226) (end 119.3292 90.4748) (width 0.2) (layer "F.Cu") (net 31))
 (segment (start 121.177 96.271228) (end 121.177 92.3226) (width 0.2) (layer "F.Cu") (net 31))
 (segment (start 123.885572 98.9798) (end 121.177 96.271228) (width 0.2) (layer "F.Cu") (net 31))
 (segment (start 125.5442 98.9798) (end 123.885572 98.9798) (width 0.2) (layer "F.Cu") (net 31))
 (segment (start 121.0754 111.5886) (end 119.3292 113.3348) (width 0.2) (layer "F.Cu") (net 39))
 (segment (start 125.5442 104.8298) (end 123.885572 104.8298) (width 0.2) (layer "F.Cu") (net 39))
 (segment (start 121.0754 107.639972) (end 121.0754 111.5886) (width 0.2) (layer "F.Cu") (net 39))
 (segment (start 123.885572 104.8298) (end 121.0754 107.639972) (width 0.2) (layer "F.Cu") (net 39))
 (segment (start 120.6754 107.474286) (end 120.6754 109.4486) (width 0.2) (layer "F.Cu") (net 38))
 (segment (start 120.6754 109.4486) (end 119.3292 110.7948) (width 0.2) (layer "F.Cu") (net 38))
 (segment (start 125.5442 104.1798) (end 123.969886 104.1798) (width 0.2) (layer "F.Cu") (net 38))
 (segment (start 123.969886 104.1798) (end 120.6754 107.474286) (width 0.2) (layer "F.Cu") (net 38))
 (segment (start 123.969886 99.6298) (end 120.777 96.436914) (width 0.2) (layer "F.Cu") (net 32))
 (segment (start 125.5442 99.6298) (end 123.969886 99.6298) (width 0.2) (layer "F.Cu") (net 32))
 (segment (start 120.777 94.4626) (end 119.3292 93.0148) (width 0.2) (layer "F.Cu") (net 32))
 (segment (start 120.777 96.436914) (end 120.777 94.4626) (width 0.2) (layer "F.Cu") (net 32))
 (segment (start 125.5442 101.5798) (end 120.2742 101.5798) (width 0.2) (layer "F.Cu") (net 34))
 (segment (start 120.2742 101.5798) (end 119.3292 100.6348) (width 0.2) (layer "F.Cu") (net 34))
 (segment (start 125.5442 100.9298) (end 122.1642 100.9298) (width 0.2) (layer "F.Cu") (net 33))
 (segment (start 122.1642 100.9298) (end 119.3292 98.0948) (width 0.2) (layer "F.Cu") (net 33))
 (segment (start 120.2742 102.2298) (end 119.3292 103.1748) (width 0.2) (layer "F.Cu") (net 35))
 (segment (start 125.5442 102.2298) (end 120.2742 102.2298) (width 0.2) (layer "F.Cu") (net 35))
 (segment (start 124.0542 103.5298) (end 125.5442 103.5298) (width 0.2) (layer "F.Cu") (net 37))
 (segment (start 119.3292 108.2548) (end 124.0542 103.5298) (width 0.2) (layer "F.Cu") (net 37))
 (segment (start 122.1642 102.8798) (end 119.3292 105.7148) (width 0.2) (layer "F.Cu") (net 36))
 (segment (start 125.5442 102.8798) (end 122.1642 102.8798) (width 0.2) (layer "F.Cu") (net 36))
 (segment (start 131.2692 103.5298) (end 132.3842 103.5298) (width 0.2) (layer "F.Cu") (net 42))
 (segment (start 132.3842 103.5298) (end 137.1092 108.2548) (width 0.2) (layer "F.Cu") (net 42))
 (segment (start 131.2692 101.5798) (end 136.1642 101.5798) (width 0.2) (layer "F.Cu") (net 45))
 (segment (start 136.1642 101.5798) (end 137.1092 100.6348) (width 0.2) (layer "F.Cu") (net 45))
 (segment (start 132.3842 100.2798) (end 137.1092 95.5548) (width 0.2) (layer "F.Cu") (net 47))
 (segment (start 131.2692 100.2798) (end 132.3842 100.2798) (width 0.2) (layer "F.Cu") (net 47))
 (segment (start 135.6868 107.398086) (end 135.6868 109.3724) (width 0.2) (layer "F.Cu") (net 41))
 (segment (start 135.6868 109.3724) (end 137.1092 110.7948) (width 0.2) (layer "F.Cu") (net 41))
 (segment (start 131.2692 104.1798) (end 132.468514 104.1798) (width 0.2) (layer "F.Cu") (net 41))
 (segment (start 132.468514 104.1798) (end 135.6868 107.398086) (width 0.2) (layer "F.Cu") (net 41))
 (segment (start 131.2692 102.8798) (end 134.2742 102.8798) (width 0.2) (layer "F.Cu") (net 43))
 (segment (start 134.2742 102.8798) (end 137.1092 105.7148) (width 0.2) (layer "F.Cu") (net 43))
 (segment (start 134.2742 100.9298) (end 137.1092 98.0948) (width 0.2) (layer "F.Cu") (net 46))
 (segment (start 131.2692 100.9298) (end 134.2742 100.9298) (width 0.2) (layer "F.Cu") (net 46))
 (segment (start 135.636 96.462314) (end 135.636 94.488) (width 0.2) (layer "F.Cu") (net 48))
 (segment (start 131.2692 99.6298) (end 132.468514 99.6298) (width 0.2) (layer "F.Cu") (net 48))
 (segment (start 132.468514 99.6298) (end 135.636 96.462314) (width 0.2) (layer "F.Cu") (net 48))
 (segment (start 135.636 94.488) (end 137.1092 93.0148) (width 0.2) (layer "F.Cu") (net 48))
 (segment (start 131.2692 102.2298) (end 136.1642 102.2298) (width 0.2) (layer "F.Cu") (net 44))
 (segment (start 136.1642 102.2298) (end 137.1092 103.1748) (width 0.2) (layer "F.Cu") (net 44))
 (segment (start 135.236 96.296628) (end 135.236 92.348) (width 0.2) (layer "F.Cu") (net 49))
 (segment (start 132.552828 98.9798) (end 135.236 96.296628) (width 0.2) (layer "F.Cu") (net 49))
 (segment (start 135.236 92.348) (end 137.1092 90.4748) (width 0.2) (layer "F.Cu") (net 49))
 (segment (start 131.2692 98.9798) (end 132.552828 98.9798) (width 0.2) (layer "F.Cu") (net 49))
 (segment (start 120.5738 142.5702) (end 119.3292 143.8148) (width 0.2) (layer "F.Cu") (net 11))
 (segment (start 123.412386 137.7573) (end 120.5738 140.595886) (width 0.2) (layer "F.Cu") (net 11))
 (segment (start 125.3567 137.7573) (end 123.412386 137.7573) (width 0.2) (layer "F.Cu") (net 11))
 (segment (start 120.5738 140.595886) (end 120.5738 142.5702) (width 0.2) (layer "F.Cu") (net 11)))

